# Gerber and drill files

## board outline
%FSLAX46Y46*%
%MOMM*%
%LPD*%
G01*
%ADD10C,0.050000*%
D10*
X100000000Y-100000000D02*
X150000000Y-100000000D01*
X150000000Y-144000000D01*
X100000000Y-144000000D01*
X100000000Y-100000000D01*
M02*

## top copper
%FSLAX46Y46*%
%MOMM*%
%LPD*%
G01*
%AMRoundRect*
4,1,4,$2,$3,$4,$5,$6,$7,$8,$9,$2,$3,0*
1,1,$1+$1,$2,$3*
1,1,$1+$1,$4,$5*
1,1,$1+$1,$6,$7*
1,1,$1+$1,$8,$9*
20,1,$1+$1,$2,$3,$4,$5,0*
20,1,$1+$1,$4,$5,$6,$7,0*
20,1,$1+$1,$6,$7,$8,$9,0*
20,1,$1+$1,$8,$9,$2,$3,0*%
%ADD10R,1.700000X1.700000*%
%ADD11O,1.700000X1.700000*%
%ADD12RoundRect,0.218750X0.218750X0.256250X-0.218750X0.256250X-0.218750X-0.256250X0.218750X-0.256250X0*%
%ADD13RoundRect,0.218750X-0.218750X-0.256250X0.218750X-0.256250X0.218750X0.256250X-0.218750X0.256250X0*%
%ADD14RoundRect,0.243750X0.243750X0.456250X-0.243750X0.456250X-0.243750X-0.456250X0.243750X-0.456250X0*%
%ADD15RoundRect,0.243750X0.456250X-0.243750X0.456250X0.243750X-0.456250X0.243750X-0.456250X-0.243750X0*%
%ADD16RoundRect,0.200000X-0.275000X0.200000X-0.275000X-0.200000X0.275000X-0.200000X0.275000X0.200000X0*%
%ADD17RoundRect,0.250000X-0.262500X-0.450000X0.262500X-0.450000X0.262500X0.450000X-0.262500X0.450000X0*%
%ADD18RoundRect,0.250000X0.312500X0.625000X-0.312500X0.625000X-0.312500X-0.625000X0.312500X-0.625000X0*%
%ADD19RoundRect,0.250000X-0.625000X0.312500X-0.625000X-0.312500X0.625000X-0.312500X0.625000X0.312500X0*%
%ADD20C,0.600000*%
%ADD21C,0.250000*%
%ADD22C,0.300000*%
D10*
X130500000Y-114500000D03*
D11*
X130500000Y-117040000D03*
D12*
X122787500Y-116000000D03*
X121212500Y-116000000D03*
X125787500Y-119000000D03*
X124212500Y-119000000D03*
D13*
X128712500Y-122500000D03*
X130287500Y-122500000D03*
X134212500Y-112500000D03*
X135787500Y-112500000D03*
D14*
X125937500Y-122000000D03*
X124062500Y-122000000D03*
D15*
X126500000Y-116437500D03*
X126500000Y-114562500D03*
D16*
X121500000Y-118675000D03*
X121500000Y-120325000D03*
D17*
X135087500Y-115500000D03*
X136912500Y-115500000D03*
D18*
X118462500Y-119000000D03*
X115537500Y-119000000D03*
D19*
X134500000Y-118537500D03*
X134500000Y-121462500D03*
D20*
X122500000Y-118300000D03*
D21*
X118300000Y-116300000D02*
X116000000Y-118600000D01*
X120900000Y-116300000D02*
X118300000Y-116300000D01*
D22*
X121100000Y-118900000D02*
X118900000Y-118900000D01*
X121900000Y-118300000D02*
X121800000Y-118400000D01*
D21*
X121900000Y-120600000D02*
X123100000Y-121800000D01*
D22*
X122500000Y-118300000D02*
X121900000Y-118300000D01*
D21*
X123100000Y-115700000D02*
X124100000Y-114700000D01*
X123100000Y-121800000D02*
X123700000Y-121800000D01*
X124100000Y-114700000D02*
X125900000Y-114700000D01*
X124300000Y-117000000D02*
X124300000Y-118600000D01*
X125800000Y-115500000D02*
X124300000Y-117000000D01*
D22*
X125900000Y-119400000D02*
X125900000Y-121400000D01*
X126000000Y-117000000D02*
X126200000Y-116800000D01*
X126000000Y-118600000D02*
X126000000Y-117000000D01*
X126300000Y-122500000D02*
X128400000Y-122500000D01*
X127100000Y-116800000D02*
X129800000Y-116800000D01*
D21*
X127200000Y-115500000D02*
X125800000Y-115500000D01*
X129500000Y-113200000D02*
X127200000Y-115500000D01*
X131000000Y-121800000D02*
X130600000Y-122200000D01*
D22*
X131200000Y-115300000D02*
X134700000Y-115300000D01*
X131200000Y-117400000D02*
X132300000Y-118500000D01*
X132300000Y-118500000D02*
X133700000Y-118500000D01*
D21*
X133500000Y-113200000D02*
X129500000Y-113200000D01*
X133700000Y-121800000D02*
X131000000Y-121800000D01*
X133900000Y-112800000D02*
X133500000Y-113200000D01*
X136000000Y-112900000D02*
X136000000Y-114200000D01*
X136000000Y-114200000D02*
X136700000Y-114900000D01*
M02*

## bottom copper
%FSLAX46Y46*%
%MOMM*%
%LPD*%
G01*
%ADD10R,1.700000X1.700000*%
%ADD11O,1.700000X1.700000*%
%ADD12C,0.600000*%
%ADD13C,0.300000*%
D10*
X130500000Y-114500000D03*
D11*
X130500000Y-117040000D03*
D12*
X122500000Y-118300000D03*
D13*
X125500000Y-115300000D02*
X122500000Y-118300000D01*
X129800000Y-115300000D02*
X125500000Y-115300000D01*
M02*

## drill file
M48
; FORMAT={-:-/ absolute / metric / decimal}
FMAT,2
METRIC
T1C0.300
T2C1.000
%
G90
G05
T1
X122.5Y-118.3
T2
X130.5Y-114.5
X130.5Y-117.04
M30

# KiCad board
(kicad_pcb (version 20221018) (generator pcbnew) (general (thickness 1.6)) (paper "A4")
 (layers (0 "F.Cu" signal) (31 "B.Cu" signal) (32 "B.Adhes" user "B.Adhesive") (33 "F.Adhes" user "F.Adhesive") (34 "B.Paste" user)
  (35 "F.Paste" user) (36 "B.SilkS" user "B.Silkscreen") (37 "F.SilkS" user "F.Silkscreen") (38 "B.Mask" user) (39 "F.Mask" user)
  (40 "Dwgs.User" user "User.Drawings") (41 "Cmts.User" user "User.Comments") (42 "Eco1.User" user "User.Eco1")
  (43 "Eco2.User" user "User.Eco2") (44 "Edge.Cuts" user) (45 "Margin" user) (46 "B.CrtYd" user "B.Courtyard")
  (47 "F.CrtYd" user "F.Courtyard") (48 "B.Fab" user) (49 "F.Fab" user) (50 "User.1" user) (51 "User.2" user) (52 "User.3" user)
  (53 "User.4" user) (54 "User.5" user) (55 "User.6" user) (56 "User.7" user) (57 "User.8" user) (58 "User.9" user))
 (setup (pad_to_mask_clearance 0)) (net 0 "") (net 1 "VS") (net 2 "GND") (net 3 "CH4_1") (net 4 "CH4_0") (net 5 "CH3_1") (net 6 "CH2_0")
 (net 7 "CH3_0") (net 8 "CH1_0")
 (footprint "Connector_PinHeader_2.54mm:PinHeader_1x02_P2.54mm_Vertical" (layer "F.Cu") (at 130.5 114.5)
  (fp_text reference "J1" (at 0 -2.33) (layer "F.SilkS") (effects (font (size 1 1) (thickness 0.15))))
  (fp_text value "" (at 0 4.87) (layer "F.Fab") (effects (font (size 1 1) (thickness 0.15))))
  (pad "1" thru_hole rect (at 0 0) (size 1.7 1.7) (drill 1) (layers "*.Cu" "*.Mask") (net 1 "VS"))
  (pad "2" thru_hole oval (at 0 2.54) (size 1.7 1.7) (drill 1) (layers "*.Cu" "*.Mask") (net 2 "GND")))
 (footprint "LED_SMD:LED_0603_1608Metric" (layer "F.Cu") (at 122 116 180)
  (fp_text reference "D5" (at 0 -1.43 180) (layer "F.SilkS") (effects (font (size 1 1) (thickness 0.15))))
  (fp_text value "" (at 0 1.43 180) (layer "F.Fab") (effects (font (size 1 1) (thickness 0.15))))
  (pad "1" smd roundrect (at -0.7875 0 180) (size 0.875 0.95) (layers "F.Cu" "F.Paste" "F.Mask") (roundrect_rratio 0.25) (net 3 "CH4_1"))
  (pad "2" smd roundrect (at 0.7875 0 180) (size 0.875 0.95) (layers "F.Cu" "F.Paste" "F.Mask") (roundrect_rratio 0.25) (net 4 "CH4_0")))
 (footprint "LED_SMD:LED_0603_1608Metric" (layer "F.Cu") (at 125 119 180)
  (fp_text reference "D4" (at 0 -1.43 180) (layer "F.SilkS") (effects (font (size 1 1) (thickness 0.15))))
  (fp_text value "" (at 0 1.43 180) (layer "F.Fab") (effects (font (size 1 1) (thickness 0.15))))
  (pad "1" smd roundrect (at -0.7875 0 180) (size 0.875 0.95) (layers "F.Cu" "F.Paste" "F.Mask") (roundrect_rratio 0.25) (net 2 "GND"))
  (pad "2" smd roundrect (at 0.7875 0 180) (size 0.875 0.95) (layers "F.Cu" "F.Paste" "F.Mask") (roundrect_rratio 0.25) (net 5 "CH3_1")))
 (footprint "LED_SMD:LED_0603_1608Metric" (layer "F.Cu") (at 129.5 122.5)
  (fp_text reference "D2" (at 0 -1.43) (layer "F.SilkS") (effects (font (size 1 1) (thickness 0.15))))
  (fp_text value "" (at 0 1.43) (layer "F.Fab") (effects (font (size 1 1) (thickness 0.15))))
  (pad "1" smd roundrect (at -0.7875 0) (size 0.875 0.95) (layers "F.Cu" "F.Paste" "F.Mask") (roundrect_rratio 0.25) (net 2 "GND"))
  (pad "2" smd roundrect (at 0.7875 0) (size 0.875 0.95) (layers "F.Cu" "F.Paste" "F.Mask") (roundrect_rratio 0.25) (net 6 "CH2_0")))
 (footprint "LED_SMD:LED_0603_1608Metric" (layer "F.Cu") (at 135 112.5)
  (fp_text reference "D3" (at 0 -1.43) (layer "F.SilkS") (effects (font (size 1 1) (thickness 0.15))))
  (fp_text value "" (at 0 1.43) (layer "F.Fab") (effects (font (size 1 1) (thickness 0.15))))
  (pad "1" smd roundrect (at -0.7875 0) (size 0.875 0.95) (layers "F.Cu" "F.Paste" "F.Mask") (roundrect_rratio 0.25) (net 5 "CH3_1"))
  (pad "2" smd roundrect (at 0.7875 0) (size 0.875 0.95) (layers "F.Cu" "F.Paste" "F.Mask") (roundrect_rratio 0.25) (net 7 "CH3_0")))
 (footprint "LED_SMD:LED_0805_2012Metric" (layer "F.Cu") (at 125 122 180)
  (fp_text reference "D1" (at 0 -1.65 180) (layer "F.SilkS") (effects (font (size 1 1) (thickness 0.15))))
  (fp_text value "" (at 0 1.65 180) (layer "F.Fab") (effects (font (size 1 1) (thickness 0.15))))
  (pad "1" smd roundrect (at -0.9375 0 180) (size 0.975 1.4) (layers "F.Cu" "F.Paste" "F.Mask") (roundrect_rratio 0.25) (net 2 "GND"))
  (pad "2" smd roundrect (at 0.9375 0 180) (size 0.975 1.4) (layers "F.Cu" "F.Paste" "F.Mask") (roundrect_rratio 0.25) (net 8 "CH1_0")))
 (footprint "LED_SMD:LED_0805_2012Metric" (layer "F.Cu") (at 126.5 115.5 90)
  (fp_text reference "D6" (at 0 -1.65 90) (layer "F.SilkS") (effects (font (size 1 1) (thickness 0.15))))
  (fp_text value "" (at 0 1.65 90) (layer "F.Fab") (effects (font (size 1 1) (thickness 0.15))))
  (pad "1" smd roundrect (at -0.9375 0 90) (size 0.975 1.4) (layers "F.Cu" "F.Paste" "F.Mask") (roundrect_rratio 0.25) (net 2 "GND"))
  (pad "2" smd roundrect (at 0.9375 0 90) (size 0.975 1.4) (layers "F.Cu" "F.Paste" "F.Mask") (roundrect_rratio 0.25) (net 3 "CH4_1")))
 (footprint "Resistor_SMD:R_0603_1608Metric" (layer "F.Cu") (at 121.5 119.5 -90)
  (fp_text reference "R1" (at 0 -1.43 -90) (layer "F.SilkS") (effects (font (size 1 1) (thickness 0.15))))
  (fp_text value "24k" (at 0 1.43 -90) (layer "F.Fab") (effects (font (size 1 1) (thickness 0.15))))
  (pad "1" smd roundrect (at -0.825 0 270) (size 0.8 0.95) (layers "F.Cu" "F.Paste" "F.Mask") (roundrect_rratio 0.25) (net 1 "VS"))
  (pad "2" smd roundrect (at 0.825 0 270) (size 0.8 0.95) (layers "F.Cu" "F.Paste" "F.Mask") (roundrect_rratio 0.25) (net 8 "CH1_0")))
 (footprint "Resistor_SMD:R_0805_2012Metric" (layer "F.Cu") (at 136 115.5)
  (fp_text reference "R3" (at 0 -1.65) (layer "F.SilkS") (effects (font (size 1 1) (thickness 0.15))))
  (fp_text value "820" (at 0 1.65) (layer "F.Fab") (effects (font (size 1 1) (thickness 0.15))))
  (pad "1" smd roundrect (at -0.9125 0) (size 1.025 1.4) (layers "F.Cu" "F.Paste" "F.Mask") (roundrect_rratio 0.243902) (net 1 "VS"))
  (pad "2" smd roundrect (at 0.9125 0) (size 1.025 1.4) (layers "F.Cu" "F.Paste" "F.Mask") (roundrect_rratio 0.243902) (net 7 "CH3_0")))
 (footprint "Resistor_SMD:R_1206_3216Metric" (layer "F.Cu") (at 117 119 180)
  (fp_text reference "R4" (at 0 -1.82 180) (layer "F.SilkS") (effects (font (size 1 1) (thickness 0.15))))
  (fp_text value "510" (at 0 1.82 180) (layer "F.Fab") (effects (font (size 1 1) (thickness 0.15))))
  (pad "1" smd roundrect (at -1.4625 0 180) (size 1.125 1.75) (layers "F.Cu" "F.Paste" "F.Mask") (roundrect_rratio 0.222222) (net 1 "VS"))
  (pad "2" smd roundrect (at 1.4625 0 180) (size 1.125 1.75) (layers "F.Cu" "F.Paste" "F.Mask") (roundrect_rratio 0.222222) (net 4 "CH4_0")))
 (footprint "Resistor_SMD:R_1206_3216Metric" (layer "F.Cu") (at 134.5 120 -90)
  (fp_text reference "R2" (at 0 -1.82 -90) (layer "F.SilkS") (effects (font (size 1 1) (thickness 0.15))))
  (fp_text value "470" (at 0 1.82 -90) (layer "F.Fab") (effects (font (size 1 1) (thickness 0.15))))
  (pad "1" smd roundrect (at -1.4625 0 270) (size 1.125 1.75) (layers "F.Cu" "F.Paste" "F.Mask") (roundrect_rratio 0.222222) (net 2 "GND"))
  (pad "2" smd roundrect (at 1.4625 0 270) (size 1.125 1.75) (layers "F.Cu" "F.Paste" "F.Mask") (roundrect_rratio 0.222222) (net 6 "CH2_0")))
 (gr_rect (start 100 100) (end 150 144) (stroke (width 0.05) (type default)) (fill none) (layer "Edge.Cuts"))
 (segment (start 118.3 116.3) (end 116 118.6) (width 0.25) (layer "F.Cu") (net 4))
 (segment (start 120.9 116.3) (end 118.3 116.3) (width 0.25) (layer "F.Cu") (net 4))
 (segment (start 121.1 118.9) (end 118.9 118.9) (width 0.3) (layer "F.Cu") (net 1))
 (segment (start 121.9 118.3) (end 121.8 118.4) (width 0.3) (layer "F.Cu") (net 1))
 (segment (start 121.9 120.6) (end 123.1 121.8) (width 0.25) (layer "F.Cu") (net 8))
 (segment (start 122.5 118.3) (end 121.9 118.3) (width 0.3) (layer "F.Cu") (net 1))
 (segment (start 123.1 115.7) (end 124.1 114.7) (width 0.25) (layer "F.Cu") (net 3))
 (segment (start 123.1 121.8) (end 123.7 121.8) (width 0.25) (layer "F.Cu") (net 8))
 (segment (start 124.1 114.7) (end 125.9 114.7) (width 0.25) (layer "F.Cu") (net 3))
 (segment (start 124.3 117) (end 124.3 118.6) (width 0.25) (layer "F.Cu") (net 5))
 (segment (start 125.8 115.5) (end 124.3 117) (width 0.25) (layer "F.Cu") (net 5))
 (segment (start 125.9 119.4) (end 125.9 121.4) (width 0.3) (layer "F.Cu") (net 2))
 (segment (start 126 117) (end 126.2 116.8) (width 0.3) (layer "F.Cu") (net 2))
 (segment (start 126 118.6) (end 126 117) (width 0.3) (layer "F.Cu") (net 2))
 (segment (start 126.3 122.5) (end 128.4 122.5) (width 0.3) (layer "F.Cu") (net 2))
 (segment (start 127.1 116.8) (end 129.8 116.8) (width 0.3) (layer "F.Cu") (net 2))
 (segment (start 127.2 115.5) (end 125.8 115.5) (width 0.25) (layer "F.Cu") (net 5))
 (segment (start 129.5 113.2) (end 127.2 115.5) (width 0.25) (layer "F.Cu") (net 5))
 (segment (start 131 121.8) (end 130.6 122.2) (width 0.25) (layer "F.Cu") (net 6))
 (segment (start 131.2 115.3) (end 134.7 115.3) (width 0.3) (layer "F.Cu") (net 1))
 (segment (start 131.2 117.4) (end 132.3 118.5) (width 0.3) (layer "F.Cu") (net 2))
 (segment (start 132.3 118.5) (end 133.7 118.5) (width 0.3) (layer "F.Cu") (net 2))
 (segment (start 133.5 113.2) (end 129.5 113.2) (width 0.25) (layer "F.Cu") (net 5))
 (segment (start 133.7 121.8) (end 131 121.8) (width 0.25) (layer "F.Cu") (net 6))
 (segment (start 133.9 112.8) (end 133.5 113.2) (width 0.25) (layer "F.Cu") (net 5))
 (segment (start 136 112.9) (end 136 114.2) (width 0.25) (layer "F.Cu") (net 7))
 (segment (start 136 114.2) (end 136.7 114.9) (width 0.25) (layer "F.Cu") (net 7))
 (via (at 122.5 118.3) (size 0.6) (drill 0.3) (layers "F.Cu" "B.Cu") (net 1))
 (segment (start 125.5 115.3) (end 122.5 118.3) (width 0.3) (layer "B.Cu") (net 1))
 (segment (start 129.8 115.3) (end 125.5 115.3) (width 0.3) (layer "B.Cu") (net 1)))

